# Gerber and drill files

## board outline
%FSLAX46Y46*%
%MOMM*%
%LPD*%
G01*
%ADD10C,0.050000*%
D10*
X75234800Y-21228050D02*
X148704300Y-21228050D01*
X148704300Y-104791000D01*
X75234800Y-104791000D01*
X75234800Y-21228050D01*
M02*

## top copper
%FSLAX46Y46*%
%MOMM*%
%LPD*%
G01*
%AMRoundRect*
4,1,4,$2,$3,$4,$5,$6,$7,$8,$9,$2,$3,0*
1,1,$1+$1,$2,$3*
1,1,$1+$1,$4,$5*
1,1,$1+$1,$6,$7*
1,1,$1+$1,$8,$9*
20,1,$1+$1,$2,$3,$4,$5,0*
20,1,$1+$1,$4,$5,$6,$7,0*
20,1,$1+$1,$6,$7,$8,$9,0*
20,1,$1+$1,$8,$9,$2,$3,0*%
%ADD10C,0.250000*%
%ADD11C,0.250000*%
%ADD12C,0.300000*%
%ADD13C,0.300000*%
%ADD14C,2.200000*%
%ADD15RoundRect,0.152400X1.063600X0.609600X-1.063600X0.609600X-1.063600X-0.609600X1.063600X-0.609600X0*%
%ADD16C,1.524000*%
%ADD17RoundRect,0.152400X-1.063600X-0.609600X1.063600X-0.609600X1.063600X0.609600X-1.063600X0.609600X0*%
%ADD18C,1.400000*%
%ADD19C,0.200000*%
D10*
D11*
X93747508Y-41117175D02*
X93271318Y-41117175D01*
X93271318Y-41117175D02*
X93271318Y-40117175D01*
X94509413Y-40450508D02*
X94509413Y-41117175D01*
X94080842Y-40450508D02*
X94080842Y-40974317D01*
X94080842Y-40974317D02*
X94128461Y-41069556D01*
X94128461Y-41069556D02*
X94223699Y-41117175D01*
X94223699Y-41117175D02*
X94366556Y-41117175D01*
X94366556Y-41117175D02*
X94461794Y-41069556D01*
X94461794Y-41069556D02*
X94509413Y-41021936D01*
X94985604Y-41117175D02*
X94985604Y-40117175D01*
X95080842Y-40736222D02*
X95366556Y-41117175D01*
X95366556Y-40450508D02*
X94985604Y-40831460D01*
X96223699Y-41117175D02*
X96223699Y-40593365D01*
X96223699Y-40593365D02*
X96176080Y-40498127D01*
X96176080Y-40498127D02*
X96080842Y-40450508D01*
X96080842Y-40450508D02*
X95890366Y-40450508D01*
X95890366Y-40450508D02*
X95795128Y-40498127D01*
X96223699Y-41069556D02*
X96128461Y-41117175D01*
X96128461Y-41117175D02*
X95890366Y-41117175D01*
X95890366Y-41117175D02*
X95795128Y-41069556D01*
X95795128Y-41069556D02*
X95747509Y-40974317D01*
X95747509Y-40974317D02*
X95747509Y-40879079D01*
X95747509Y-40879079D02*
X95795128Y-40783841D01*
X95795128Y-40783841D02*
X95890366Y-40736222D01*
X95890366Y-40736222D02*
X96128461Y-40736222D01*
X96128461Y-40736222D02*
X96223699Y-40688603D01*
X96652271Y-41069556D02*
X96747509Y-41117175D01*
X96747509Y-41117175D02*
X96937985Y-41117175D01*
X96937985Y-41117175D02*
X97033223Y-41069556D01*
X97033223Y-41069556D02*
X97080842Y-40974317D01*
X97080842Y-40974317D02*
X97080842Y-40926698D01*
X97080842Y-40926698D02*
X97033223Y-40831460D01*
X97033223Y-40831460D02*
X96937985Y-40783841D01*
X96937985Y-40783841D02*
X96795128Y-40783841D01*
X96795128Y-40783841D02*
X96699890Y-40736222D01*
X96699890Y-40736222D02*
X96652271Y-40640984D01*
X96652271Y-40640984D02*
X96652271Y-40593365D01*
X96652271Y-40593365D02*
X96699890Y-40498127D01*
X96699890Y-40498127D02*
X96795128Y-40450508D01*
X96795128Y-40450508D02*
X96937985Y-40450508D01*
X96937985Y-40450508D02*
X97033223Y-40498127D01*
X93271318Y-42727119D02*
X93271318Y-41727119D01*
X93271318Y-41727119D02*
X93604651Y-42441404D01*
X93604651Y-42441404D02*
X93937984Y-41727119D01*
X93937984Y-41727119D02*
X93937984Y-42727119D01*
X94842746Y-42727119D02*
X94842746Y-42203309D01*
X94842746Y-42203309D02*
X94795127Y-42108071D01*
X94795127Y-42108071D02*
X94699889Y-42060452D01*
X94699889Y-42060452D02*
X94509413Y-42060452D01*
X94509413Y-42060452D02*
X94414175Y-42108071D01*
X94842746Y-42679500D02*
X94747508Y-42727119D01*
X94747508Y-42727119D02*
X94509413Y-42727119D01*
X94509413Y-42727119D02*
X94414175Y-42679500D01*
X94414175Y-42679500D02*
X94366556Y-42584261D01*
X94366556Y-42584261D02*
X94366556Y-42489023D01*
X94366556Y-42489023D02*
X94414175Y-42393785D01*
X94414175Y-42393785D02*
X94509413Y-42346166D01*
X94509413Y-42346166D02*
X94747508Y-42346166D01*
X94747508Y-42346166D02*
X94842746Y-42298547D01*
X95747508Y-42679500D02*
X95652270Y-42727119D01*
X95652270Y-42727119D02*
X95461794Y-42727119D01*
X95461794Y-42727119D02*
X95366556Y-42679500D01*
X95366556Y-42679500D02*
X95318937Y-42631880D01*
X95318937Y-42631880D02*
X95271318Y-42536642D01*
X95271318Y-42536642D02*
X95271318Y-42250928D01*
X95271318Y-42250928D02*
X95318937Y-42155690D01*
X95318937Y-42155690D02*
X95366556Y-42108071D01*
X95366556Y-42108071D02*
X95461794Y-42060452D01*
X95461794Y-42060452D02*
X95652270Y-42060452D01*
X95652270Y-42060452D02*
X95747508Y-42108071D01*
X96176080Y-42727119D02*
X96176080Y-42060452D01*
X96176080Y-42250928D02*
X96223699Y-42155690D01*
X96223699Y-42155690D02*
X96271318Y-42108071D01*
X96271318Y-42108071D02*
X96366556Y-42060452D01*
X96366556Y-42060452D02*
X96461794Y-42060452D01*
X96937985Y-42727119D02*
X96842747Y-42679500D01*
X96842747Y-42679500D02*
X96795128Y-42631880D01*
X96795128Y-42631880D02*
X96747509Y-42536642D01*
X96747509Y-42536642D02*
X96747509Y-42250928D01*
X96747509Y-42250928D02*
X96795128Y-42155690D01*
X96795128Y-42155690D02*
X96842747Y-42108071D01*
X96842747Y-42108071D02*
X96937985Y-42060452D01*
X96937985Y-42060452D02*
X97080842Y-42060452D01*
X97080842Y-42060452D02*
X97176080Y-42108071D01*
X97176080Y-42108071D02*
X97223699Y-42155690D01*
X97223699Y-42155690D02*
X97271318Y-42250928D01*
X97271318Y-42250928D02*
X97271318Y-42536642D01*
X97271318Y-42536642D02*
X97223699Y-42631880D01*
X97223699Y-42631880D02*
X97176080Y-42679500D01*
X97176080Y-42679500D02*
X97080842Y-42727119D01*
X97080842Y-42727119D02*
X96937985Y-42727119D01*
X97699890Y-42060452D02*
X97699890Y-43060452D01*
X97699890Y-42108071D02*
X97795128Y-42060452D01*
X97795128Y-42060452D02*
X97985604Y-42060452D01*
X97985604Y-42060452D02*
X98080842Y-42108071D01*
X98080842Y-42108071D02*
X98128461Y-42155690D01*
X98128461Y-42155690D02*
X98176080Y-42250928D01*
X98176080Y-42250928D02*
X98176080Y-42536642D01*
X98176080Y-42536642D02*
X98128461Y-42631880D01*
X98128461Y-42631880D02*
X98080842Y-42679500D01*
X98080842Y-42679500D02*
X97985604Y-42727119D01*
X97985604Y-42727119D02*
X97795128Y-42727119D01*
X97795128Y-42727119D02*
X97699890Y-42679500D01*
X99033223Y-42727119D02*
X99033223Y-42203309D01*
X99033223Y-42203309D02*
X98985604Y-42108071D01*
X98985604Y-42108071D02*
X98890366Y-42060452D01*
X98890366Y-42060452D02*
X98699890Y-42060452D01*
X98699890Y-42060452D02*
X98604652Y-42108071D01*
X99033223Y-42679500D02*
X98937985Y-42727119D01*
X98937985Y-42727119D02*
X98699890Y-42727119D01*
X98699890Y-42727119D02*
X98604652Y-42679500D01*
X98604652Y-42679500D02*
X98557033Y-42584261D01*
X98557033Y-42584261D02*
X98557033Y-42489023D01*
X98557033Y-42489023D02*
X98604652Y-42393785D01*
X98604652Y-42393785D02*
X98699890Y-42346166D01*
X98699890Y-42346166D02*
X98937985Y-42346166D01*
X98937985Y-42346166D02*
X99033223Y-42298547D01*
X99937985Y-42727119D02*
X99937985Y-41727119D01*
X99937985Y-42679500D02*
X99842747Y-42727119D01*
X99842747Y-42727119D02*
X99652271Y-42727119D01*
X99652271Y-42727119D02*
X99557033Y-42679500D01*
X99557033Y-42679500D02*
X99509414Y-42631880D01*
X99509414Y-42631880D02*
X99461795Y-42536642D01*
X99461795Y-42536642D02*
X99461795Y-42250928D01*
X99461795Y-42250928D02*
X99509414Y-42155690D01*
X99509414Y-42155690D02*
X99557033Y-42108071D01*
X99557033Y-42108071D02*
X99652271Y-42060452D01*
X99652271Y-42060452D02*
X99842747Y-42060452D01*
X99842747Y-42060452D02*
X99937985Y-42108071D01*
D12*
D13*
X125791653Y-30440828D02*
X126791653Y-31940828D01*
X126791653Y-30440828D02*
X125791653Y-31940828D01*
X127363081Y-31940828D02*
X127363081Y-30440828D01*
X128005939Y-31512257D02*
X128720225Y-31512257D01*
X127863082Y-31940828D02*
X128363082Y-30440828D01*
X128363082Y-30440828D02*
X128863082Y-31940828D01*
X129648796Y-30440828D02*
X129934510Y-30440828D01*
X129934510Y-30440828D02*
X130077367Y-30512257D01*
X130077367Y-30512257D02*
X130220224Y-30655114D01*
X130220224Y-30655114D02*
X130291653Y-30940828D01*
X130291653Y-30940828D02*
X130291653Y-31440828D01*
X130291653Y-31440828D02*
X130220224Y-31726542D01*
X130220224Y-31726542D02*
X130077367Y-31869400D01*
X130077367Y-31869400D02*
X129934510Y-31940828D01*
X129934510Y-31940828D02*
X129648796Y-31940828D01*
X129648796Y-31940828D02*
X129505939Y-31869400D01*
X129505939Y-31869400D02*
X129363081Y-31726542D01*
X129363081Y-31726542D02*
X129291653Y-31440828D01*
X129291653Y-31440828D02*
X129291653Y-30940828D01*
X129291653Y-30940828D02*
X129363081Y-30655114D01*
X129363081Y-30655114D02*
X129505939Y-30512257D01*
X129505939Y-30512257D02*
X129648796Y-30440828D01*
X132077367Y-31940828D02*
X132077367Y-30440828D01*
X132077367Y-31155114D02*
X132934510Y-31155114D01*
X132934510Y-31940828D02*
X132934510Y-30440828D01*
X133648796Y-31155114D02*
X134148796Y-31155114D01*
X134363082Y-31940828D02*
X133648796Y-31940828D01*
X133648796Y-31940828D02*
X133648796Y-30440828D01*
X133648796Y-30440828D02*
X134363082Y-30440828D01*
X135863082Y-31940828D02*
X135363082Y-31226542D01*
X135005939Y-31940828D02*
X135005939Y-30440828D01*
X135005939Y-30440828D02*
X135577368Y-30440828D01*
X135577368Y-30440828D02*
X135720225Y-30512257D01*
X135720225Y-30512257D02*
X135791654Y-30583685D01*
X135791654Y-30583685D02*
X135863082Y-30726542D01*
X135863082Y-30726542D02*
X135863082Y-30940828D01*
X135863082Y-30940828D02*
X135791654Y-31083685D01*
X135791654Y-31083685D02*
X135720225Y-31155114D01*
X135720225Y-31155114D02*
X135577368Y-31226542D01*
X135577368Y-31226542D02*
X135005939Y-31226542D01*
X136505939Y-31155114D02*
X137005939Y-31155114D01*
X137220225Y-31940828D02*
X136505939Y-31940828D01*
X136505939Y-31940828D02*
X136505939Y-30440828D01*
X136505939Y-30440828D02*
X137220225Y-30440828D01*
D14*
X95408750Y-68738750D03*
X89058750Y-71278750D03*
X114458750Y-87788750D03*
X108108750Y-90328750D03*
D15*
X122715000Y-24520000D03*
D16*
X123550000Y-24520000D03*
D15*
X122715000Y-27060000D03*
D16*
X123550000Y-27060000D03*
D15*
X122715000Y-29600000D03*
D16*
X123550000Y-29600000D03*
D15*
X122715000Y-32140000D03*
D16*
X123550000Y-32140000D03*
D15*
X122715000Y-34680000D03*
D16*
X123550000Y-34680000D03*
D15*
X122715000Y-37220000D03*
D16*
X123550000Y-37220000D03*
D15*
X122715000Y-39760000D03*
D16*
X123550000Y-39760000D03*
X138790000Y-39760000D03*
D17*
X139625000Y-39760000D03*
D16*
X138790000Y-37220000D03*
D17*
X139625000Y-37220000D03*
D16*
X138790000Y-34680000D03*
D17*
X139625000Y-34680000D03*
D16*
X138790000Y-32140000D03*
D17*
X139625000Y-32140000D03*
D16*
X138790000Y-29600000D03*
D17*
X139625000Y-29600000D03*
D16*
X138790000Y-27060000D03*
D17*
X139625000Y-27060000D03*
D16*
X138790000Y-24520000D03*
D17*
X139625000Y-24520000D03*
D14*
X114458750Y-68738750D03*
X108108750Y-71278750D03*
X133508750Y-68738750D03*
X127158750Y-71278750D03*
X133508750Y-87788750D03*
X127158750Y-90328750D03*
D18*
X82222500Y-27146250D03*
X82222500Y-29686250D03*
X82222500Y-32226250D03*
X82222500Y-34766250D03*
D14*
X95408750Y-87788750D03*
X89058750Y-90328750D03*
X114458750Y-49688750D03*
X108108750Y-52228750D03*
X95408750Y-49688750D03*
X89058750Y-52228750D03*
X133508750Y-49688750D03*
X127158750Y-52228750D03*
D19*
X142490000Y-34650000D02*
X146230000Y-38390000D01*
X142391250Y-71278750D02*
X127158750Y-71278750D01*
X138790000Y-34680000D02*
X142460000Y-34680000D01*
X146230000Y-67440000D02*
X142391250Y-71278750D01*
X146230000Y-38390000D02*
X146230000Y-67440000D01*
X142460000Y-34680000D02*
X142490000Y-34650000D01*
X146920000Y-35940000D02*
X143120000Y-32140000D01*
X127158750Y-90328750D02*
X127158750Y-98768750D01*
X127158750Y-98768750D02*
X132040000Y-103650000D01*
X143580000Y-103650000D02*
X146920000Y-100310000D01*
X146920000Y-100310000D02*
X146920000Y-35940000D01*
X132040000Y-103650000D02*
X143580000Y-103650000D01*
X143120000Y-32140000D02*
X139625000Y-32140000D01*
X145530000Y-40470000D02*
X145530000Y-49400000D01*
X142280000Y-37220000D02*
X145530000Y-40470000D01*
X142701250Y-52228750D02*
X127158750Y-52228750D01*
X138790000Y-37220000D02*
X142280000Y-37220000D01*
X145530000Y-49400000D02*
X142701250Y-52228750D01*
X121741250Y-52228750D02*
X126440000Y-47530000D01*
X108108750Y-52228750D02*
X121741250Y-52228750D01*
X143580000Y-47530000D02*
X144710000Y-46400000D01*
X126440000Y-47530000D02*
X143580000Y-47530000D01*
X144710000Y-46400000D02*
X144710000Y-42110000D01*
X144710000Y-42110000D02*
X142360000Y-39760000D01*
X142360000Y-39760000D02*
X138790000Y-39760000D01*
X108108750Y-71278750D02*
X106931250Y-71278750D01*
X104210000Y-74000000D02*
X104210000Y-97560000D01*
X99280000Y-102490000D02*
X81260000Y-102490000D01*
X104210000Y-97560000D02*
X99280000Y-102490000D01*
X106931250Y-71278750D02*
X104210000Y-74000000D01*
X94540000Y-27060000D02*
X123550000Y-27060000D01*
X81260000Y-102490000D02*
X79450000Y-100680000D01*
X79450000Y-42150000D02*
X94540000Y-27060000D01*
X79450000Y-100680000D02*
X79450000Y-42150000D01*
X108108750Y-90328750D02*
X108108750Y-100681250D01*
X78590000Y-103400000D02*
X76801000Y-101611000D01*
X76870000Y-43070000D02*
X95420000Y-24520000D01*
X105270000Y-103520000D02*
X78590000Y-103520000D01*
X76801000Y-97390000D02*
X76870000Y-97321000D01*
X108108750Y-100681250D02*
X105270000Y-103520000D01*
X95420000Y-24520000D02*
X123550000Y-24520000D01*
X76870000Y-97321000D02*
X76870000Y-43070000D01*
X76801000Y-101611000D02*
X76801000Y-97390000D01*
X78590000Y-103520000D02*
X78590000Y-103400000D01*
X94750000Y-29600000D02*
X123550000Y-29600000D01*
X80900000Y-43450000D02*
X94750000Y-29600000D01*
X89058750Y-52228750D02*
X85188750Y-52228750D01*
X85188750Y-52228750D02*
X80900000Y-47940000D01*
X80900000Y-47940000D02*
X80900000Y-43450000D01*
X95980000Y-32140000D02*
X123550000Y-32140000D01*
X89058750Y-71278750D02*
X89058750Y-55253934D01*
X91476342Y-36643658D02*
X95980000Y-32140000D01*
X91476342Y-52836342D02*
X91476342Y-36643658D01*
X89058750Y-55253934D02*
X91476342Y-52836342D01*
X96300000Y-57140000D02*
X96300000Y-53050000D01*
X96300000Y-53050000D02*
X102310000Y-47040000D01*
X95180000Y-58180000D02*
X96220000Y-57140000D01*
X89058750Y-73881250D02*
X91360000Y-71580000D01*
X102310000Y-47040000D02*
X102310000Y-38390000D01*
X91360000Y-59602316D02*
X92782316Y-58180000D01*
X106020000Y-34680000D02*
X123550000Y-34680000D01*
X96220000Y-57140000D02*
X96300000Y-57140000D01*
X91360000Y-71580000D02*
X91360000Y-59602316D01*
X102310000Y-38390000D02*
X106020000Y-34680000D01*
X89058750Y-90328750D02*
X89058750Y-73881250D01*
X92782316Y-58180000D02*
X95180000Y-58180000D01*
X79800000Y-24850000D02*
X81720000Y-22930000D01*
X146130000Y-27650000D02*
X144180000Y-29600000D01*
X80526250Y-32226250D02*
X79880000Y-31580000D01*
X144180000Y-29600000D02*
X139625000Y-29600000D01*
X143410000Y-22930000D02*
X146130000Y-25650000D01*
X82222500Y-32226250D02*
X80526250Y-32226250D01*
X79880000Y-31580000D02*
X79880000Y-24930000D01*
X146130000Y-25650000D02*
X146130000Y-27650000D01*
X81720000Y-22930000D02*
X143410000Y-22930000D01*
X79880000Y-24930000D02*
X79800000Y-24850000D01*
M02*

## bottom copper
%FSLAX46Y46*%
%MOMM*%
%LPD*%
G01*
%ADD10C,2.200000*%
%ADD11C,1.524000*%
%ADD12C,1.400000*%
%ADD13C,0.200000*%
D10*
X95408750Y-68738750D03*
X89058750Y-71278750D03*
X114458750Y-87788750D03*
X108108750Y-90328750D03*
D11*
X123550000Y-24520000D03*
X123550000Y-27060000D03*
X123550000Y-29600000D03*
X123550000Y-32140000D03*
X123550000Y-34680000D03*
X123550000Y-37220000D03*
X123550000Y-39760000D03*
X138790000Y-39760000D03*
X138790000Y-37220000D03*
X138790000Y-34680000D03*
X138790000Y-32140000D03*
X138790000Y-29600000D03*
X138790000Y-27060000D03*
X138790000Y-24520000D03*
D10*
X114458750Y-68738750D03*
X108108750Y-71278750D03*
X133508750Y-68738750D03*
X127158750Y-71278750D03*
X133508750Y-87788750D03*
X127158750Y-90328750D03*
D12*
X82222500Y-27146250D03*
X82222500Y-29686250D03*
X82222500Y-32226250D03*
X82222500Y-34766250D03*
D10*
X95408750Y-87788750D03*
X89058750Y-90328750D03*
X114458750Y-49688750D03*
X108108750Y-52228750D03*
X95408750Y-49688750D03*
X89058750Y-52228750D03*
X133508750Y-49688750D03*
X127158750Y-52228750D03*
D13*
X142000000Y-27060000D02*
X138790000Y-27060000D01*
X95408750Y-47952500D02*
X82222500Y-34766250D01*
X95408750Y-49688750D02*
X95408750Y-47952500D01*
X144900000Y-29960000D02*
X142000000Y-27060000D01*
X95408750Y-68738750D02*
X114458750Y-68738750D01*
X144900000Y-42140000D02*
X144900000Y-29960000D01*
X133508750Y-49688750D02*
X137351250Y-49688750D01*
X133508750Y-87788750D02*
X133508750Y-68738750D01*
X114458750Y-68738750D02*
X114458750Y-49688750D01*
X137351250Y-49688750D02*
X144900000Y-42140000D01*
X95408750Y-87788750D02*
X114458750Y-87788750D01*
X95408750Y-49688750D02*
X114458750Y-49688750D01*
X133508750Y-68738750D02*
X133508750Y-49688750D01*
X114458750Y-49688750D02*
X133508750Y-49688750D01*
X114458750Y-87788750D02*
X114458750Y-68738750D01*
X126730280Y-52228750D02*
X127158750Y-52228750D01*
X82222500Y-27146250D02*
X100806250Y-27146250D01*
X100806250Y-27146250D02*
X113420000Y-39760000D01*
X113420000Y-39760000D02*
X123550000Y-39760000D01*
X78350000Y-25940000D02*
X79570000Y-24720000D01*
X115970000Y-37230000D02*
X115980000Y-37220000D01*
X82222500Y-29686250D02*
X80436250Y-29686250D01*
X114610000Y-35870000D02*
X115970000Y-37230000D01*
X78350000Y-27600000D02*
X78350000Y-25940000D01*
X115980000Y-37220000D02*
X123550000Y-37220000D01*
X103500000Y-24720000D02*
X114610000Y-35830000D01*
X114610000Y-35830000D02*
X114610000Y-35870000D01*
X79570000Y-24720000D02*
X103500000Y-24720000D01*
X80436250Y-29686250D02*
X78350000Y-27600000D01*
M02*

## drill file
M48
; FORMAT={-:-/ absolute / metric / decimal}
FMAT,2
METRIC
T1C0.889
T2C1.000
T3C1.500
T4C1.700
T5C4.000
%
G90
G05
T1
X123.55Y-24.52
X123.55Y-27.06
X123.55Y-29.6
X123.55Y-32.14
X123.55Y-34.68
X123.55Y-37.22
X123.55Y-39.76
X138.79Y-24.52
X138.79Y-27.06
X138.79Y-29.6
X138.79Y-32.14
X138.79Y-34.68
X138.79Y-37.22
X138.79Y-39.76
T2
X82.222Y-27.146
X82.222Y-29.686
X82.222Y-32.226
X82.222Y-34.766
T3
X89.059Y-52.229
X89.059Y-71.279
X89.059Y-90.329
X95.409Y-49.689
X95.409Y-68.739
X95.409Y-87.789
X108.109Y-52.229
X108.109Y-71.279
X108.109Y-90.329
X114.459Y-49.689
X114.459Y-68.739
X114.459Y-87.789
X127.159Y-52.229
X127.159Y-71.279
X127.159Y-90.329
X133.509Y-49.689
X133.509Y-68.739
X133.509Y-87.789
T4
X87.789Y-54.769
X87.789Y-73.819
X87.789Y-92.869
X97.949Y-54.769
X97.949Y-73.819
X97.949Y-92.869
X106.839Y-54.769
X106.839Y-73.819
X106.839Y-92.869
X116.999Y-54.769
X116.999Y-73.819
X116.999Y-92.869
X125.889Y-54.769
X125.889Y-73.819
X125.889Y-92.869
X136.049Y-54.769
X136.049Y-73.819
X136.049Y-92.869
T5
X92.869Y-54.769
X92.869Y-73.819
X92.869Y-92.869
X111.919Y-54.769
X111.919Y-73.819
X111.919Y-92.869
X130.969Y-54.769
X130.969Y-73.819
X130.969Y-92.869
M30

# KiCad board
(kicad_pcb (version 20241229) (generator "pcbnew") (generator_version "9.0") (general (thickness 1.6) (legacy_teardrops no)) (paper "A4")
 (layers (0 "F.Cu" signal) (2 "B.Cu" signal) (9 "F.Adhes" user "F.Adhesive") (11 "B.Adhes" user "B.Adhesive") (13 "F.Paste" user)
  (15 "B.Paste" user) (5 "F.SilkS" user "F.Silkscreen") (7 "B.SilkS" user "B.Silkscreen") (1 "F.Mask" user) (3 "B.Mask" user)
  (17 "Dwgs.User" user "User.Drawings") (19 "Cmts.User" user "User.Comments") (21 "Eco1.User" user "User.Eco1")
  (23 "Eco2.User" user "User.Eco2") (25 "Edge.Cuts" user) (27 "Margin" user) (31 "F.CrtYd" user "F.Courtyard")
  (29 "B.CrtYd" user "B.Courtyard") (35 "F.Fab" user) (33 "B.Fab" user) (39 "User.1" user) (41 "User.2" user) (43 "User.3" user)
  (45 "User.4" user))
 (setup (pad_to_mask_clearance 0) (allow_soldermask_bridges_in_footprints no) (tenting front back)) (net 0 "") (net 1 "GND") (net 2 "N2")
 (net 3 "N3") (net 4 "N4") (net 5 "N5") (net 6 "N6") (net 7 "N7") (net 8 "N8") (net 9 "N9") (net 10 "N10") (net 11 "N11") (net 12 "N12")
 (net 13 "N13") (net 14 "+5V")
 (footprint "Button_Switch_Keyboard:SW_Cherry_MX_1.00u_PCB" (layer "F.Cu") (at 95.40875 68.73875)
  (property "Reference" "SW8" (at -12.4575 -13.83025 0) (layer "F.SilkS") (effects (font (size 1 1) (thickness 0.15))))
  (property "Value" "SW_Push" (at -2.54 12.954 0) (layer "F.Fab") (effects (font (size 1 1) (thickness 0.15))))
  (pad "" np_thru_hole circle (at -7.62 5.08) (size 1.7 1.7) (drill 1.7) (layers "*.Cu" "*.Mask"))
  (pad "" np_thru_hole circle (at -2.54 5.08) (size 4 4) (drill 4) (layers "*.Cu" "*.Mask"))
  (pad "" np_thru_hole circle (at 2.54 5.08) (size 1.7 1.7) (drill 1.7) (layers "*.Cu" "*.Mask"))
  (pad "1" thru_hole circle (at 0 0) (size 2.2 2.2) (drill 1.5) (layers "*.Cu" "*.Mask") (remove_unused_layers no) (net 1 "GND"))
  (pad "2" thru_hole circle (at -6.35 2.54) (size 2.2 2.2) (drill 1.5) (layers "*.Cu" "*.Mask") (remove_unused_layers no) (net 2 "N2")))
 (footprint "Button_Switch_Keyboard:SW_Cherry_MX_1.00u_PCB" (layer "F.Cu") (at 114.45875 87.78875)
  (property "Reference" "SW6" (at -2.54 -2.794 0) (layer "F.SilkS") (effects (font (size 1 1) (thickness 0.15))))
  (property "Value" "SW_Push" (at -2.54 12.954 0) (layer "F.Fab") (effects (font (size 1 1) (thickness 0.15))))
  (pad "" np_thru_hole circle (at -7.62 5.08) (size 1.7 1.7) (drill 1.7) (layers "*.Cu" "*.Mask"))
  (pad "" np_thru_hole circle (at -2.54 5.08) (size 4 4) (drill 4) (layers "*.Cu" "*.Mask"))
  (pad "" np_thru_hole circle (at 2.54 5.08) (size 1.7 1.7) (drill 1.7) (layers "*.Cu" "*.Mask"))
  (pad "1" thru_hole circle (at 0 0) (size 2.2 2.2) (drill 1.5) (layers "*.Cu" "*.Mask") (remove_unused_layers no) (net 1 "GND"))
  (pad "2" thru_hole circle (at -6.35 2.54) (size 2.2 2.2) (drill 1.5) (layers "*.Cu" "*.Mask") (remove_unused_layers no) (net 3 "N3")))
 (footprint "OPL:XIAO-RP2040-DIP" (layer "F.Cu") (at 131.17 32.14)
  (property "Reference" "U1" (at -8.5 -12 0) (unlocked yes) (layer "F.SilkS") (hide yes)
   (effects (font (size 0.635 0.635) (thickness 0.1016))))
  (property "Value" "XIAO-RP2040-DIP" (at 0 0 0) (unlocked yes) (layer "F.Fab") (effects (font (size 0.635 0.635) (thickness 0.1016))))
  (pad "1" smd roundrect (at -8.455 -7.62 180) (size 2.432 1.524) (layers "F.Cu" "F.Mask") (roundrect_rratio 0.1) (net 3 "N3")
   (thermal_bridge_angle 45))
  (pad "1" thru_hole circle (at -7.62 -7.62 180) (size 1.524 1.524) (drill 0.889) (layers "*.Cu" "*.Mask") (remove_unused_layers no)
   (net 3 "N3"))
  (pad "2" smd roundrect (at -8.455 -5.08 180) (size 2.432 1.524) (layers "F.Cu" "F.Mask") (roundrect_rratio 0.1) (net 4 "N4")
   (thermal_bridge_angle 45))
  (pad "2" thru_hole circle (at -7.62 -5.08 180) (size 1.524 1.524) (drill 0.889) (layers "*.Cu" "*.Mask") (remove_unused_layers no)
   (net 4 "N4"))
  (pad "3" smd roundrect (at -8.455 -2.54 180) (size 2.432 1.524) (layers "F.Cu" "F.Mask") (roundrect_rratio 0.1) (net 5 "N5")
   (thermal_bridge_angle 45))
  (pad "3" thru_hole circle (at -7.62 -2.54 180) (size 1.524 1.524) (drill 0.889) (layers "*.Cu" "*.Mask") (remove_unused_layers no)
   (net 5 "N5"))
  (pad "4" smd roundrect (at -8.455 0 180) (size 2.432 1.524) (layers "F.Cu" "F.Mask") (roundrect_rratio 0.1) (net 2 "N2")
   (thermal_bridge_angle 45))
  (pad "4" thru_hole circle (at -7.62 0 180) (size 1.524 1.524) (drill 0.889) (layers "*.Cu" "*.Mask") (remove_unused_layers no)
   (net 2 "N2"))
  (pad "5" smd roundrect (at -8.455 2.54 180) (size 2.432 1.524) (layers "F.Cu" "F.Mask") (roundrect_rratio 0.1) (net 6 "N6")
   (thermal_bridge_angle 45))
  (pad "5" thru_hole circle (at -7.62 2.54 180) (size 1.524 1.524) (drill 0.889) (layers "*.Cu" "*.Mask") (remove_unused_layers no)
   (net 6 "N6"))
  (pad "6" smd roundrect (at -8.455 5.08 180) (size 2.432 1.524) (layers "F.Cu" "F.Mask") (roundrect_rratio 0.1) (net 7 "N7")
   (thermal_bridge_angle 45))
  (pad "6" thru_hole circle (at -7.62 5.08 180) (size 1.524 1.524) (drill 0.889) (layers "*.Cu" "*.Mask") (remove_unused_layers no)
   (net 7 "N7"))
  (pad "7" smd roundrect (at -8.455 7.62 180) (size 2.432 1.524) (layers "F.Cu" "F.Mask") (roundrect_rratio 0.1) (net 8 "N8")
   (thermal_bridge_angle 45))
  (pad "7" thru_hole circle (at -7.62 7.62 180) (size 1.524 1.524) (drill 0.889) (layers "*.Cu" "*.Mask") (remove_unused_layers no)
   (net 8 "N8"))
  (pad "8" thru_hole circle (at 7.62 7.62) (size 1.524 1.524) (drill 0.889) (layers "*.Cu" "*.Mask") (remove_unused_layers no) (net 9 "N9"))
  (pad "8" smd roundrect (at 8.455 7.62) (size 2.432 1.524) (layers "F.Cu" "F.Mask") (roundrect_rratio 0.1) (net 9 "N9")
   (thermal_bridge_angle 45))
  (pad "9" thru_hole circle (at 7.62 5.08) (size 1.524 1.524) (drill 0.889) (layers "*.Cu" "*.Mask") (remove_unused_layers no)
   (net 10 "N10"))
  (pad "9" smd roundrect (at 8.455 5.08) (size 2.432 1.524) (layers "F.Cu" "F.Mask") (roundrect_rratio 0.1) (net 10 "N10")
   (thermal_bridge_angle 45))
  (pad "10" thru_hole circle (at 7.62 2.54) (size 1.524 1.524) (drill 0.889) (layers "*.Cu" "*.Mask") (remove_unused_layers no)
   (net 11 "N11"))
  (pad "10" smd roundrect (at 8.455 2.54) (size 2.432 1.524) (layers "F.Cu" "F.Mask") (roundrect_rratio 0.1) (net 11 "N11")
   (thermal_bridge_angle 45))
  (pad "11" thru_hole circle (at 7.62 0) (size 1.524 1.524) (drill 0.889) (layers "*.Cu" "*.Mask") (remove_unused_layers no) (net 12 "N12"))
  (pad "11" smd roundrect (at 8.455 0) (size 2.432 1.524) (layers "F.Cu" "F.Mask") (roundrect_rratio 0.1) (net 12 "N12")
   (thermal_bridge_angle 45))
  (pad "12" thru_hole circle (at 7.62 -2.54) (size 1.524 1.524) (drill 0.889) (layers "*.Cu" "*.Mask") (remove_unused_layers no)
   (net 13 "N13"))
  (pad "12" smd roundrect (at 8.455 -2.54) (size 2.432 1.524) (layers "F.Cu" "F.Mask") (roundrect_rratio 0.1) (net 13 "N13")
   (thermal_bridge_angle 45))
  (pad "13" thru_hole circle (at 7.62 -5.08) (size 1.524 1.524) (drill 0.889) (layers "*.Cu" "*.Mask") (remove_unused_layers no)
   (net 1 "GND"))
  (pad "13" smd roundrect (at 8.455 -5.08) (size 2.432 1.524) (layers "F.Cu" "F.Mask") (roundrect_rratio 0.1) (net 1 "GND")
   (thermal_bridge_angle 45))
  (pad "14" thru_hole circle (at 7.62 -7.62) (size 1.524 1.524) (drill 0.889) (layers "*.Cu" "*.Mask") (remove_unused_layers no)
   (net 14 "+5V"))
  (pad "14" smd roundrect (at 8.455 -7.62) (size 2.432 1.524) (layers "F.Cu" "F.Mask") (roundrect_rratio 0.1) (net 14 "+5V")
   (thermal_bridge_angle 45)))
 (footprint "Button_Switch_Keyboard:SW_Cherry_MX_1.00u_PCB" (layer "F.Cu") (at 114.45875 68.73875)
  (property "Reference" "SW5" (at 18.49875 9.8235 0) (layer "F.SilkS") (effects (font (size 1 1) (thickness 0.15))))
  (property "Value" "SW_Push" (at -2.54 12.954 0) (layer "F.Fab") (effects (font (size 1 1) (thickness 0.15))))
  (pad "" np_thru_hole circle (at -7.62 5.08) (size 1.7 1.7) (drill 1.7) (layers "*.Cu" "*.Mask"))
  (pad "" np_thru_hole circle (at -2.54 5.08) (size 4 4) (drill 4) (layers "*.Cu" "*.Mask"))
  (pad "" np_thru_hole circle (at 2.54 5.08) (size 1.7 1.7) (drill 1.7) (layers "*.Cu" "*.Mask"))
  (pad "1" thru_hole circle (at 0 0) (size 2.2 2.2) (drill 1.5) (layers "*.Cu" "*.Mask") (remove_unused_layers no) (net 1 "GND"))
  (pad "2" thru_hole circle (at -6.35 2.54) (size 2.2 2.2) (drill 1.5) (layers "*.Cu" "*.Mask") (remove_unused_layers no) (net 4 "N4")))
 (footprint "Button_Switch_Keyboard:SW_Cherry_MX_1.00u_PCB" (layer "F.Cu") (at 133.50875 68.73875)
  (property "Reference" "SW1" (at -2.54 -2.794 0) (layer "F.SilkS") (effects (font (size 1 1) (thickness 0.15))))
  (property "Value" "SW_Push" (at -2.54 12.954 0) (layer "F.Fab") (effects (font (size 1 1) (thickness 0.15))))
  (pad "" np_thru_hole circle (at -7.62 5.08) (size 1.7 1.7) (drill 1.7) (layers "*.Cu" "*.Mask"))
  (pad "" np_thru_hole circle (at -2.54 5.08) (size 4 4) (drill 4) (layers "*.Cu" "*.Mask"))
  (pad "" np_thru_hole circle (at 2.54 5.08) (size 1.7 1.7) (drill 1.7) (layers "*.Cu" "*.Mask"))
  (pad "1" thru_hole circle (at 0 0) (size 2.2 2.2) (drill 1.5) (layers "*.Cu" "*.Mask") (remove_unused_layers no) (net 1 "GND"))
  (pad "2" thru_hole circle (at -6.35 2.54) (size 2.2 2.2) (drill 1.5) (layers "*.Cu" "*.Mask") (remove_unused_layers no) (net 11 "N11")))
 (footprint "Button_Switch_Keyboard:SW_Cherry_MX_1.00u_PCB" (layer "F.Cu") (at 133.50875 87.78875)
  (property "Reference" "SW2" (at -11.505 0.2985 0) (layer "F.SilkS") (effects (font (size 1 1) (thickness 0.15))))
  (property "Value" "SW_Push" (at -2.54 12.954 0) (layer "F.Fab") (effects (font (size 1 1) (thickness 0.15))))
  (pad "" np_thru_hole circle (at -7.62 5.08) (size 1.7 1.7) (drill 1.7) (layers "*.Cu" "*.Mask"))
  (pad "" np_thru_hole circle (at -2.54 5.08) (size 4 4) (drill 4) (layers "*.Cu" "*.Mask"))
  (pad "" np_thru_hole circle (at 2.54 5.08) (size 1.7 1.7) (drill 1.7) (layers "*.Cu" "*.Mask"))
  (pad "1" thru_hole circle (at 0 0) (size 2.2 2.2) (drill 1.5) (layers "*.Cu" "*.Mask") (remove_unused_layers no) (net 1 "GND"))
  (pad "2" thru_hole circle (at -6.35 2.54) (size 2.2 2.2) (drill 1.5) (layers "*.Cu" "*.Mask") (remove_unused_layers no) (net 12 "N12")))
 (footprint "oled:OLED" (layer "F.Cu") (at 82.2225 30.95625 -90)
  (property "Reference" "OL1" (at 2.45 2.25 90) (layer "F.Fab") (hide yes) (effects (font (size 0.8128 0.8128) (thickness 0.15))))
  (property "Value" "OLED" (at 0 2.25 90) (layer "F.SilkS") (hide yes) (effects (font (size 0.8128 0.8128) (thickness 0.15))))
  (pad "1" thru_hole circle (at -3.81 0 270) (size 1.4 1.4) (drill 1) (layers "*.Cu" "*.Mask") (remove_unused_layers no) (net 8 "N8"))
  (pad "2" thru_hole circle (at -1.27 0 270) (size 1.4 1.4) (drill 1) (layers "*.Cu" "*.Mask") (remove_unused_layers no) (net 7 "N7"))
  (pad "3" thru_hole circle (at 1.27 0 270) (size 1.4 1.4) (drill 1) (layers "*.Cu" "*.Mask") (remove_unused_layers no) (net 13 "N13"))
  (pad "4" thru_hole circle (at 3.81 0 270) (size 1.4 1.4) (drill 1) (layers "*.Cu" "*.Mask") (remove_unused_layers no) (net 1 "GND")))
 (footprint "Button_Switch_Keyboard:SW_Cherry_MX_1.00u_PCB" (layer "F.Cu") (at 95.40875 87.78875)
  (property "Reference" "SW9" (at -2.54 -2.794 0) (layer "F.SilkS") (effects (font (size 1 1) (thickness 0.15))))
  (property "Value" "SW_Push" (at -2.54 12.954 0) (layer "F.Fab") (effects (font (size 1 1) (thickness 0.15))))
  (pad "" np_thru_hole circle (at -7.62 5.08) (size 1.7 1.7) (drill 1.7) (layers "*.Cu" "*.Mask"))
  (pad "" np_thru_hole circle (at -2.54 5.08) (size 4 4) (drill 4) (layers "*.Cu" "*.Mask"))
  (pad "" np_thru_hole circle (at 2.54 5.08) (size 1.7 1.7) (drill 1.7) (layers "*.Cu" "*.Mask"))
  (pad "1" thru_hole circle (at 0 0) (size 2.2 2.2) (drill 1.5) (layers "*.Cu" "*.Mask") (remove_unused_layers no) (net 1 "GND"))
  (pad "2" thru_hole circle (at -6.35 2.54) (size 2.2 2.2) (drill 1.5) (layers "*.Cu" "*.Mask") (remove_unused_layers no) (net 6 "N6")))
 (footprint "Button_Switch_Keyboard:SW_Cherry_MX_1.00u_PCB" (layer "F.Cu") (at 114.45875 49.68875)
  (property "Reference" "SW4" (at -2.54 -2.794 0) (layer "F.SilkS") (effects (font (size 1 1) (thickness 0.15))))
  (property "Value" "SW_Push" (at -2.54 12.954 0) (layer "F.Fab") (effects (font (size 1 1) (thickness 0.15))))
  (pad "" np_thru_hole circle (at -7.62 5.08) (size 1.7 1.7) (drill 1.7) (layers "*.Cu" "*.Mask"))
  (pad "" np_thru_hole circle (at -2.54 5.08) (size 4 4) (drill 4) (layers "*.Cu" "*.Mask"))
  (pad "" np_thru_hole circle (at 2.54 5.08) (size 1.7 1.7) (drill 1.7) (layers "*.Cu" "*.Mask"))
  (pad "1" thru_hole circle (at 0 0) (size 2.2 2.2) (drill 1.5) (layers "*.Cu" "*.Mask") (remove_unused_layers no) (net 1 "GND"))
  (pad "2" thru_hole circle (at -6.35 2.54) (size 2.2 2.2) (drill 1.5) (layers "*.Cu" "*.Mask") (remove_unused_layers no) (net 9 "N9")))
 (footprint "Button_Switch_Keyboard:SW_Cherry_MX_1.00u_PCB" (layer "F.Cu") (at 95.40875 49.68875)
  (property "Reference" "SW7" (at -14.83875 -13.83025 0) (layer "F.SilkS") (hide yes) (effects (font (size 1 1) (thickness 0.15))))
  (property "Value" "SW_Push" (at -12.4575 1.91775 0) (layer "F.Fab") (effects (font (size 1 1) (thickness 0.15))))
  (pad "" np_thru_hole circle (at -7.62 5.08) (size 1.7 1.7) (drill 1.7) (layers "*.Cu" "*.Mask"))
  (pad "" np_thru_hole circle (at -2.54 5.08) (size 4 4) (drill 4) (layers "*.Cu" "*.Mask"))
  (pad "" np_thru_hole circle (at 2.54 5.08) (size 1.7 1.7) (drill 1.7) (layers "*.Cu" "*.Mask"))
  (pad "1" thru_hole circle (at 0 0) (size 2.2 2.2) (drill 1.5) (layers "*.Cu" "*.Mask") (remove_unused_layers no) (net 1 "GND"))
  (pad "2" thru_hole circle (at -6.35 2.54) (size 2.2 2.2) (drill 1.5) (layers "*.Cu" "*.Mask") (remove_unused_layers no) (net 5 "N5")))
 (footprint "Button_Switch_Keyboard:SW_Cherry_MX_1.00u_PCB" (layer "F.Cu") (at 133.50875 49.68875)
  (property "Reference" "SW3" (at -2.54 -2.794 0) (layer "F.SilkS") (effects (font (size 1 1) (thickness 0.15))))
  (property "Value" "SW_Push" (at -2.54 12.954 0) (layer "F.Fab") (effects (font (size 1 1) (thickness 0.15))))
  (pad "" np_thru_hole circle (at -7.62 5.08) (size 1.7 1.7) (drill 1.7) (layers "*.Cu" "*.Mask"))
  (pad "" np_thru_hole circle (at -2.54 5.08) (size 4 4) (drill 4) (layers "*.Cu" "*.Mask"))
  (pad "" np_thru_hole circle (at 2.54 5.08) (size 1.7 1.7) (drill 1.7) (layers "*.Cu" "*.Mask"))
  (pad "1" thru_hole circle (at 0 0) (size 2.2 2.2) (drill 1.5) (layers "*.Cu" "*.Mask") (remove_unused_layers no) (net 1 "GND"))
  (pad "2" thru_hole circle (at -6.35 2.54) (size 2.2 2.2) (drill 1.5) (layers "*.Cu" "*.Mask") (remove_unused_layers no) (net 10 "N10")))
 (gr_rect (start 75.2348 21.22805) (end 148.7043 104.791) (stroke (width 0.05) (type default)) (fill no) (layer "Edge.Cuts"))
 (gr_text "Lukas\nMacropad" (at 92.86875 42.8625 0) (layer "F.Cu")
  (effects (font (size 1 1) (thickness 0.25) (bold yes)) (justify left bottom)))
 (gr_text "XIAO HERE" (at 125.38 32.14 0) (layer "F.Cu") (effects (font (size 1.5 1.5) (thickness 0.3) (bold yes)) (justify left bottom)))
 (segment (start 142 27.06) (end 138.79 27.06) (width 0.2) (layer "B.Cu") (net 1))
 (segment (start 95.40875 47.9525) (end 82.2225 34.76625) (width 0.2) (layer "B.Cu") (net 1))
 (segment (start 95.40875 49.68875) (end 95.40875 47.9525) (width 0.2) (layer "B.Cu") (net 1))
 (segment (start 144.9 29.96) (end 142 27.06) (width 0.2) (layer "B.Cu") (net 1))
 (segment (start 95.40875 68.73875) (end 114.45875 68.73875) (width 0.2) (layer "B.Cu") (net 1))
 (segment (start 144.9 42.14) (end 144.9 29.96) (width 0.2) (layer "B.Cu") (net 1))
 (segment (start 133.50875 49.68875) (end 137.35125 49.68875) (width 0.2) (layer "B.Cu") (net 1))
 (segment (start 133.50875 87.78875) (end 133.50875 68.73875) (width 0.2) (layer "B.Cu") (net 1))
 (segment (start 114.45875 68.73875) (end 114.45875 49.68875) (width 0.2) (layer "B.Cu") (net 1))
 (segment (start 137.35125 49.68875) (end 144.9 42.14) (width 0.2) (layer "B.Cu") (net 1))
 (segment (start 95.40875 87.78875) (end 114.45875 87.78875) (width 0.2) (layer "B.Cu") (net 1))
 (segment (start 95.40875 49.68875) (end 114.45875 49.68875) (width 0.2) (layer "B.Cu") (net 1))
 (segment (start 133.50875 68.73875) (end 133.50875 49.68875) (width 0.2) (layer "B.Cu") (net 1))
 (segment (start 114.45875 49.68875) (end 133.50875 49.68875) (width 0.2) (layer "B.Cu") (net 1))
 (segment (start 114.45875 87.78875) (end 114.45875 68.73875) (width 0.2) (layer "B.Cu") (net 1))
 (segment (start 142.49 34.65) (end 146.23 38.39) (width 0.2) (layer "F.Cu") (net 11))
 (segment (start 142.39125 71.27875) (end 127.15875 71.27875) (width 0.2) (layer "F.Cu") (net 11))
 (segment (start 138.79 34.68) (end 142.46 34.68) (width 0.2) (layer "F.Cu") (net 11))
 (segment (start 146.23 67.44) (end 142.39125 71.27875) (width 0.2) (layer "F.Cu") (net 11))
 (segment (start 146.23 38.39) (end 146.23 67.44) (width 0.2) (layer "F.Cu") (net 11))
 (segment (start 142.46 34.68) (end 142.49 34.65) (width 0.2) (layer "F.Cu") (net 11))
 (segment (start 146.92 35.94) (end 143.12 32.14) (width 0.2) (layer "F.Cu") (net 12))
 (segment (start 127.15875 90.32875) (end 127.15875 98.76875) (width 0.2) (layer "F.Cu") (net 12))
 (segment (start 127.15875 98.76875) (end 132.04 103.65) (width 0.2) (layer "F.Cu") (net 12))
 (segment (start 143.58 103.65) (end 146.92 100.31) (width 0.2) (layer "F.Cu") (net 12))
 (segment (start 146.92 100.31) (end 146.92 35.94) (width 0.2) (layer "F.Cu") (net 12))
 (segment (start 132.04 103.65) (end 143.58 103.65) (width 0.2) (layer "F.Cu") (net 12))
 (segment (start 143.12 32.14) (end 139.625 32.14) (width 0.2) (layer "F.Cu") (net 12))
 (segment (start 145.53 40.47) (end 145.53 49.4) (width 0.2) (layer "F.Cu") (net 10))
 (segment (start 142.28 37.22) (end 145.53 40.47) (width 0.2) (layer "F.Cu") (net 10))
 (segment (start 142.70125 52.22875) (end 127.15875 52.22875) (width 0.2) (layer "F.Cu") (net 10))
 (segment (start 138.79 37.22) (end 142.28 37.22) (width 0.2) (layer "F.Cu") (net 10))
 (segment (start 145.53 49.4) (end 142.70125 52.22875) (width 0.2) (layer "F.Cu") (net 10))
 (segment (start 126.73028 52.22875) (end 127.15875 52.22875) (width 0.2) (layer "B.Cu") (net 10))
 (segment (start 121.74125 52.22875) (end 126.44 47.53) (width 0.2) (layer "F.Cu") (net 9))
 (segment (start 108.10875 52.22875) (end 121.74125 52.22875) (width 0.2) (layer "F.Cu") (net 9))
 (segment (start 143.58 47.53) (end 144.71 46.4) (width 0.2) (layer "F.Cu") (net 9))
 (segment (start 126.44 47.53) (end 143.58 47.53) (width 0.2) (layer "F.Cu") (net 9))
 (segment (start 144.71 46.4) (end 144.71 42.11) (width 0.2) (layer "F.Cu") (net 9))
 (segment (start 144.71 42.11) (end 142.36 39.76) (width 0.2) (layer "F.Cu") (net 9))
 (segment (start 142.36 39.76) (end 138.79 39.76) (width 0.2) (layer "F.Cu") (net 9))
 (segment (start 108.10875 71.27875) (end 106.93125 71.27875) (width 0.2) (layer "F.Cu") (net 4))
 (segment (start 104.21 74) (end 104.21 97.56) (width 0.2) (layer "F.Cu") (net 4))
 (segment (start 99.28 102.49) (end 81.26 102.49) (width 0.2) (layer "F.Cu") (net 4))
 (segment (start 104.21 97.56) (end 99.28 102.49) (width 0.2) (layer "F.Cu") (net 4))
 (segment (start 106.93125 71.27875) (end 104.21 74) (width 0.2) (layer "F.Cu") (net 4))
 (segment (start 94.54 27.06) (end 123.55 27.06) (width 0.2) (layer "F.Cu") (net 4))
 (segment (start 81.26 102.49) (end 79.45 100.68) (width 0.2) (layer "F.Cu") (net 4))
 (segment (start 79.45 42.15) (end 94.54 27.06) (width 0.2) (layer "F.Cu") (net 4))
 (segment (start 79.45 100.68) (end 79.45 42.15) (width 0.2) (layer "F.Cu") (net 4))
 (segment (start 108.10875 90.32875) (end 108.10875 100.68125) (width 0.2) (layer "F.Cu") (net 3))
 (segment (start 78.59 103.4) (end 76.801 101.611) (width 0.2) (layer "F.Cu") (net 3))
 (segment (start 76.87 43.07) (end 95.42 24.52) (width 0.2) (layer "F.Cu") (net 3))
 (segment (start 105.27 103.52) (end 78.59 103.52) (width 0.2) (layer "F.Cu") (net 3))
 (segment (start 76.801 97.39) (end 76.87 97.321) (width 0.2) (layer "F.Cu") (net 3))
 (segment (start 108.10875 100.68125) (end 105.27 103.52) (width 0.2) (layer "F.Cu") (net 3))
 (segment (start 95.42 24.52) (end 123.55 24.52) (width 0.2) (layer "F.Cu") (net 3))
 (segment (start 76.87 97.321) (end 76.87 43.07) (width 0.2) (layer "F.Cu") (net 3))
 (segment (start 76.801 101.611) (end 76.801 97.39) (width 0.2) (layer "F.Cu") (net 3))
 (segment (start 78.59 103.52) (end 78.59 103.4) (width 0.2) (layer "F.Cu") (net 3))
 (segment (start 94.75 29.6) (end 123.55 29.6) (width 0.2) (layer "F.Cu") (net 5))
 (segment (start 80.9 43.45) (end 94.75 29.6) (width 0.2) (layer "F.Cu") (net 5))
 (segment (start 89.05875 52.22875) (end 85.18875 52.22875) (width 0.2) (layer "F.Cu") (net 5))
 (segment (start 85.18875 52.22875) (end 80.9 47.94) (width 0.2) (layer "F.Cu") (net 5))
 (segment (start 80.9 47.94) (end 80.9 43.45) (width 0.2) (layer "F.Cu") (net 5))
 (segment (start 95.98 32.14) (end 123.55 32.14) (width 0.2) (layer "F.Cu") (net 2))
 (segment (start 89.05875 71.27875) (end 89.05875 55.253934) (width 0.2) (layer "F.Cu") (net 2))
 (segment (start 91.476342 36.643658) (end 95.98 32.14) (width 0.2) (layer "F.Cu") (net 2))
 (segment (start 91.476342 52.836342) (end 91.476342 36.643658) (width 0.2) (layer "F.Cu") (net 2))
 (segment (start 89.05875 55.253934) (end 91.476342 52.836342) (width 0.2) (layer "F.Cu") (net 2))
 (segment (start 96.3 57.14) (end 96.3 53.05) (width 0.2) (layer "F.Cu") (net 6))
 (segment (start 96.3 53.05) (end 102.31 47.04) (width 0.2) (layer "F.Cu") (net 6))
 (segment (start 95.18 58.18) (end 96.22 57.14) (width 0.2) (layer "F.Cu") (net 6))
 (segment (start 89.05875 73.88125) (end 91.36 71.58) (width 0.2) (layer "F.Cu") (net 6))
 (segment (start 102.31 47.04) (end 102.31 38.39) (width 0.2) (layer "F.Cu") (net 6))
 (segment (start 91.36 59.602316) (end 92.782316 58.18) (width 0.2) (layer "F.Cu") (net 6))
 (segment (start 106.02 34.68) (end 123.55 34.68) (width 0.2) (layer "F.Cu") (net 6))
 (segment (start 96.22 57.14) (end 96.3 57.14) (width 0.2) (layer "F.Cu") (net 6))
 (segment (start 91.36 71.58) (end 91.36 59.602316) (width 0.2) (layer "F.Cu") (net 6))
 (segment (start 102.31 38.39) (end 106.02 34.68) (width 0.2) (layer "F.Cu") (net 6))
 (segment (start 89.05875 90.32875) (end 89.05875 73.88125) (width 0.2) (layer "F.Cu") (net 6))
 (segment (start 92.782316 58.18) (end 95.18 58.18) (width 0.2) (layer "F.Cu") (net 6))
 (segment (start 82.2225 27.14625) (end 100.80625 27.14625) (width 0.2) (layer "B.Cu") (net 8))
 (segment (start 100.80625 27.14625) (end 113.42 39.76) (width 0.2) (layer "B.Cu") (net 8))
 (segment (start 113.42 39.76) (end 123.55 39.76) (width 0.2) (layer "B.Cu") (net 8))
 (segment (start 79.8 24.85) (end 81.72 22.93) (width 0.2) (layer "F.Cu") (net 13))
 (segment (start 146.13 27.65) (end 144.18 29.6) (width 0.2) (layer "F.Cu") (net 13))
 (segment (start 80.52625 32.22625) (end 79.88 31.58) (width 0.2) (layer "F.Cu") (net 13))
 (segment (start 144.18 29.6) (end 139.625 29.6) (width 0.2) (layer "F.Cu") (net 13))
 (segment (start 143.41 22.93) (end 146.13 25.65) (width 0.2) (layer "F.Cu") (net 13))
 (segment (start 82.2225 32.22625) (end 80.52625 32.22625) (width 0.2) (layer "F.Cu") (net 13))
 (segment (start 79.88 31.58) (end 79.88 24.93) (width 0.2) (layer "F.Cu") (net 13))
 (segment (start 146.13 25.65) (end 146.13 27.65) (width 0.2) (layer "F.Cu") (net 13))
 (segment (start 81.72 22.93) (end 143.41 22.93) (width 0.2) (layer "F.Cu") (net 13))
 (segment (start 79.88 24.93) (end 79.8 24.85) (width 0.2) (layer "F.Cu") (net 13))
 (segment (start 78.35 25.94) (end 79.57 24.72) (width 0.2) (layer "B.Cu") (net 7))
 (segment (start 115.97 37.23) (end 115.98 37.22) (width 0.2) (layer "B.Cu") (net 7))
 (segment (start 82.2225 29.68625) (end 80.43625 29.68625) (width 0.2) (layer "B.Cu") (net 7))
 (segment (start 114.61 35.87) (end 115.97 37.23) (width 0.2) (layer "B.Cu") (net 7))
 (segment (start 78.35 27.6) (end 78.35 25.94) (width 0.2) (layer "B.Cu") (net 7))
 (segment (start 115.98 37.22) (end 123.55 37.22) (width 0.2) (layer "B.Cu") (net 7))
 (segment (start 103.5 24.72) (end 114.61 35.83) (width 0.2) (layer "B.Cu") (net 7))
 (segment (start 114.61 35.83) (end 114.61 35.87) (width 0.2) (layer "B.Cu") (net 7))
 (segment (start 79.57 24.72) (end 103.5 24.72) (width 0.2) (layer "B.Cu") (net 7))
 (segment (start 80.43625 29.68625) (end 78.35 27.6) (width 0.2) (layer "B.Cu") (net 7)))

